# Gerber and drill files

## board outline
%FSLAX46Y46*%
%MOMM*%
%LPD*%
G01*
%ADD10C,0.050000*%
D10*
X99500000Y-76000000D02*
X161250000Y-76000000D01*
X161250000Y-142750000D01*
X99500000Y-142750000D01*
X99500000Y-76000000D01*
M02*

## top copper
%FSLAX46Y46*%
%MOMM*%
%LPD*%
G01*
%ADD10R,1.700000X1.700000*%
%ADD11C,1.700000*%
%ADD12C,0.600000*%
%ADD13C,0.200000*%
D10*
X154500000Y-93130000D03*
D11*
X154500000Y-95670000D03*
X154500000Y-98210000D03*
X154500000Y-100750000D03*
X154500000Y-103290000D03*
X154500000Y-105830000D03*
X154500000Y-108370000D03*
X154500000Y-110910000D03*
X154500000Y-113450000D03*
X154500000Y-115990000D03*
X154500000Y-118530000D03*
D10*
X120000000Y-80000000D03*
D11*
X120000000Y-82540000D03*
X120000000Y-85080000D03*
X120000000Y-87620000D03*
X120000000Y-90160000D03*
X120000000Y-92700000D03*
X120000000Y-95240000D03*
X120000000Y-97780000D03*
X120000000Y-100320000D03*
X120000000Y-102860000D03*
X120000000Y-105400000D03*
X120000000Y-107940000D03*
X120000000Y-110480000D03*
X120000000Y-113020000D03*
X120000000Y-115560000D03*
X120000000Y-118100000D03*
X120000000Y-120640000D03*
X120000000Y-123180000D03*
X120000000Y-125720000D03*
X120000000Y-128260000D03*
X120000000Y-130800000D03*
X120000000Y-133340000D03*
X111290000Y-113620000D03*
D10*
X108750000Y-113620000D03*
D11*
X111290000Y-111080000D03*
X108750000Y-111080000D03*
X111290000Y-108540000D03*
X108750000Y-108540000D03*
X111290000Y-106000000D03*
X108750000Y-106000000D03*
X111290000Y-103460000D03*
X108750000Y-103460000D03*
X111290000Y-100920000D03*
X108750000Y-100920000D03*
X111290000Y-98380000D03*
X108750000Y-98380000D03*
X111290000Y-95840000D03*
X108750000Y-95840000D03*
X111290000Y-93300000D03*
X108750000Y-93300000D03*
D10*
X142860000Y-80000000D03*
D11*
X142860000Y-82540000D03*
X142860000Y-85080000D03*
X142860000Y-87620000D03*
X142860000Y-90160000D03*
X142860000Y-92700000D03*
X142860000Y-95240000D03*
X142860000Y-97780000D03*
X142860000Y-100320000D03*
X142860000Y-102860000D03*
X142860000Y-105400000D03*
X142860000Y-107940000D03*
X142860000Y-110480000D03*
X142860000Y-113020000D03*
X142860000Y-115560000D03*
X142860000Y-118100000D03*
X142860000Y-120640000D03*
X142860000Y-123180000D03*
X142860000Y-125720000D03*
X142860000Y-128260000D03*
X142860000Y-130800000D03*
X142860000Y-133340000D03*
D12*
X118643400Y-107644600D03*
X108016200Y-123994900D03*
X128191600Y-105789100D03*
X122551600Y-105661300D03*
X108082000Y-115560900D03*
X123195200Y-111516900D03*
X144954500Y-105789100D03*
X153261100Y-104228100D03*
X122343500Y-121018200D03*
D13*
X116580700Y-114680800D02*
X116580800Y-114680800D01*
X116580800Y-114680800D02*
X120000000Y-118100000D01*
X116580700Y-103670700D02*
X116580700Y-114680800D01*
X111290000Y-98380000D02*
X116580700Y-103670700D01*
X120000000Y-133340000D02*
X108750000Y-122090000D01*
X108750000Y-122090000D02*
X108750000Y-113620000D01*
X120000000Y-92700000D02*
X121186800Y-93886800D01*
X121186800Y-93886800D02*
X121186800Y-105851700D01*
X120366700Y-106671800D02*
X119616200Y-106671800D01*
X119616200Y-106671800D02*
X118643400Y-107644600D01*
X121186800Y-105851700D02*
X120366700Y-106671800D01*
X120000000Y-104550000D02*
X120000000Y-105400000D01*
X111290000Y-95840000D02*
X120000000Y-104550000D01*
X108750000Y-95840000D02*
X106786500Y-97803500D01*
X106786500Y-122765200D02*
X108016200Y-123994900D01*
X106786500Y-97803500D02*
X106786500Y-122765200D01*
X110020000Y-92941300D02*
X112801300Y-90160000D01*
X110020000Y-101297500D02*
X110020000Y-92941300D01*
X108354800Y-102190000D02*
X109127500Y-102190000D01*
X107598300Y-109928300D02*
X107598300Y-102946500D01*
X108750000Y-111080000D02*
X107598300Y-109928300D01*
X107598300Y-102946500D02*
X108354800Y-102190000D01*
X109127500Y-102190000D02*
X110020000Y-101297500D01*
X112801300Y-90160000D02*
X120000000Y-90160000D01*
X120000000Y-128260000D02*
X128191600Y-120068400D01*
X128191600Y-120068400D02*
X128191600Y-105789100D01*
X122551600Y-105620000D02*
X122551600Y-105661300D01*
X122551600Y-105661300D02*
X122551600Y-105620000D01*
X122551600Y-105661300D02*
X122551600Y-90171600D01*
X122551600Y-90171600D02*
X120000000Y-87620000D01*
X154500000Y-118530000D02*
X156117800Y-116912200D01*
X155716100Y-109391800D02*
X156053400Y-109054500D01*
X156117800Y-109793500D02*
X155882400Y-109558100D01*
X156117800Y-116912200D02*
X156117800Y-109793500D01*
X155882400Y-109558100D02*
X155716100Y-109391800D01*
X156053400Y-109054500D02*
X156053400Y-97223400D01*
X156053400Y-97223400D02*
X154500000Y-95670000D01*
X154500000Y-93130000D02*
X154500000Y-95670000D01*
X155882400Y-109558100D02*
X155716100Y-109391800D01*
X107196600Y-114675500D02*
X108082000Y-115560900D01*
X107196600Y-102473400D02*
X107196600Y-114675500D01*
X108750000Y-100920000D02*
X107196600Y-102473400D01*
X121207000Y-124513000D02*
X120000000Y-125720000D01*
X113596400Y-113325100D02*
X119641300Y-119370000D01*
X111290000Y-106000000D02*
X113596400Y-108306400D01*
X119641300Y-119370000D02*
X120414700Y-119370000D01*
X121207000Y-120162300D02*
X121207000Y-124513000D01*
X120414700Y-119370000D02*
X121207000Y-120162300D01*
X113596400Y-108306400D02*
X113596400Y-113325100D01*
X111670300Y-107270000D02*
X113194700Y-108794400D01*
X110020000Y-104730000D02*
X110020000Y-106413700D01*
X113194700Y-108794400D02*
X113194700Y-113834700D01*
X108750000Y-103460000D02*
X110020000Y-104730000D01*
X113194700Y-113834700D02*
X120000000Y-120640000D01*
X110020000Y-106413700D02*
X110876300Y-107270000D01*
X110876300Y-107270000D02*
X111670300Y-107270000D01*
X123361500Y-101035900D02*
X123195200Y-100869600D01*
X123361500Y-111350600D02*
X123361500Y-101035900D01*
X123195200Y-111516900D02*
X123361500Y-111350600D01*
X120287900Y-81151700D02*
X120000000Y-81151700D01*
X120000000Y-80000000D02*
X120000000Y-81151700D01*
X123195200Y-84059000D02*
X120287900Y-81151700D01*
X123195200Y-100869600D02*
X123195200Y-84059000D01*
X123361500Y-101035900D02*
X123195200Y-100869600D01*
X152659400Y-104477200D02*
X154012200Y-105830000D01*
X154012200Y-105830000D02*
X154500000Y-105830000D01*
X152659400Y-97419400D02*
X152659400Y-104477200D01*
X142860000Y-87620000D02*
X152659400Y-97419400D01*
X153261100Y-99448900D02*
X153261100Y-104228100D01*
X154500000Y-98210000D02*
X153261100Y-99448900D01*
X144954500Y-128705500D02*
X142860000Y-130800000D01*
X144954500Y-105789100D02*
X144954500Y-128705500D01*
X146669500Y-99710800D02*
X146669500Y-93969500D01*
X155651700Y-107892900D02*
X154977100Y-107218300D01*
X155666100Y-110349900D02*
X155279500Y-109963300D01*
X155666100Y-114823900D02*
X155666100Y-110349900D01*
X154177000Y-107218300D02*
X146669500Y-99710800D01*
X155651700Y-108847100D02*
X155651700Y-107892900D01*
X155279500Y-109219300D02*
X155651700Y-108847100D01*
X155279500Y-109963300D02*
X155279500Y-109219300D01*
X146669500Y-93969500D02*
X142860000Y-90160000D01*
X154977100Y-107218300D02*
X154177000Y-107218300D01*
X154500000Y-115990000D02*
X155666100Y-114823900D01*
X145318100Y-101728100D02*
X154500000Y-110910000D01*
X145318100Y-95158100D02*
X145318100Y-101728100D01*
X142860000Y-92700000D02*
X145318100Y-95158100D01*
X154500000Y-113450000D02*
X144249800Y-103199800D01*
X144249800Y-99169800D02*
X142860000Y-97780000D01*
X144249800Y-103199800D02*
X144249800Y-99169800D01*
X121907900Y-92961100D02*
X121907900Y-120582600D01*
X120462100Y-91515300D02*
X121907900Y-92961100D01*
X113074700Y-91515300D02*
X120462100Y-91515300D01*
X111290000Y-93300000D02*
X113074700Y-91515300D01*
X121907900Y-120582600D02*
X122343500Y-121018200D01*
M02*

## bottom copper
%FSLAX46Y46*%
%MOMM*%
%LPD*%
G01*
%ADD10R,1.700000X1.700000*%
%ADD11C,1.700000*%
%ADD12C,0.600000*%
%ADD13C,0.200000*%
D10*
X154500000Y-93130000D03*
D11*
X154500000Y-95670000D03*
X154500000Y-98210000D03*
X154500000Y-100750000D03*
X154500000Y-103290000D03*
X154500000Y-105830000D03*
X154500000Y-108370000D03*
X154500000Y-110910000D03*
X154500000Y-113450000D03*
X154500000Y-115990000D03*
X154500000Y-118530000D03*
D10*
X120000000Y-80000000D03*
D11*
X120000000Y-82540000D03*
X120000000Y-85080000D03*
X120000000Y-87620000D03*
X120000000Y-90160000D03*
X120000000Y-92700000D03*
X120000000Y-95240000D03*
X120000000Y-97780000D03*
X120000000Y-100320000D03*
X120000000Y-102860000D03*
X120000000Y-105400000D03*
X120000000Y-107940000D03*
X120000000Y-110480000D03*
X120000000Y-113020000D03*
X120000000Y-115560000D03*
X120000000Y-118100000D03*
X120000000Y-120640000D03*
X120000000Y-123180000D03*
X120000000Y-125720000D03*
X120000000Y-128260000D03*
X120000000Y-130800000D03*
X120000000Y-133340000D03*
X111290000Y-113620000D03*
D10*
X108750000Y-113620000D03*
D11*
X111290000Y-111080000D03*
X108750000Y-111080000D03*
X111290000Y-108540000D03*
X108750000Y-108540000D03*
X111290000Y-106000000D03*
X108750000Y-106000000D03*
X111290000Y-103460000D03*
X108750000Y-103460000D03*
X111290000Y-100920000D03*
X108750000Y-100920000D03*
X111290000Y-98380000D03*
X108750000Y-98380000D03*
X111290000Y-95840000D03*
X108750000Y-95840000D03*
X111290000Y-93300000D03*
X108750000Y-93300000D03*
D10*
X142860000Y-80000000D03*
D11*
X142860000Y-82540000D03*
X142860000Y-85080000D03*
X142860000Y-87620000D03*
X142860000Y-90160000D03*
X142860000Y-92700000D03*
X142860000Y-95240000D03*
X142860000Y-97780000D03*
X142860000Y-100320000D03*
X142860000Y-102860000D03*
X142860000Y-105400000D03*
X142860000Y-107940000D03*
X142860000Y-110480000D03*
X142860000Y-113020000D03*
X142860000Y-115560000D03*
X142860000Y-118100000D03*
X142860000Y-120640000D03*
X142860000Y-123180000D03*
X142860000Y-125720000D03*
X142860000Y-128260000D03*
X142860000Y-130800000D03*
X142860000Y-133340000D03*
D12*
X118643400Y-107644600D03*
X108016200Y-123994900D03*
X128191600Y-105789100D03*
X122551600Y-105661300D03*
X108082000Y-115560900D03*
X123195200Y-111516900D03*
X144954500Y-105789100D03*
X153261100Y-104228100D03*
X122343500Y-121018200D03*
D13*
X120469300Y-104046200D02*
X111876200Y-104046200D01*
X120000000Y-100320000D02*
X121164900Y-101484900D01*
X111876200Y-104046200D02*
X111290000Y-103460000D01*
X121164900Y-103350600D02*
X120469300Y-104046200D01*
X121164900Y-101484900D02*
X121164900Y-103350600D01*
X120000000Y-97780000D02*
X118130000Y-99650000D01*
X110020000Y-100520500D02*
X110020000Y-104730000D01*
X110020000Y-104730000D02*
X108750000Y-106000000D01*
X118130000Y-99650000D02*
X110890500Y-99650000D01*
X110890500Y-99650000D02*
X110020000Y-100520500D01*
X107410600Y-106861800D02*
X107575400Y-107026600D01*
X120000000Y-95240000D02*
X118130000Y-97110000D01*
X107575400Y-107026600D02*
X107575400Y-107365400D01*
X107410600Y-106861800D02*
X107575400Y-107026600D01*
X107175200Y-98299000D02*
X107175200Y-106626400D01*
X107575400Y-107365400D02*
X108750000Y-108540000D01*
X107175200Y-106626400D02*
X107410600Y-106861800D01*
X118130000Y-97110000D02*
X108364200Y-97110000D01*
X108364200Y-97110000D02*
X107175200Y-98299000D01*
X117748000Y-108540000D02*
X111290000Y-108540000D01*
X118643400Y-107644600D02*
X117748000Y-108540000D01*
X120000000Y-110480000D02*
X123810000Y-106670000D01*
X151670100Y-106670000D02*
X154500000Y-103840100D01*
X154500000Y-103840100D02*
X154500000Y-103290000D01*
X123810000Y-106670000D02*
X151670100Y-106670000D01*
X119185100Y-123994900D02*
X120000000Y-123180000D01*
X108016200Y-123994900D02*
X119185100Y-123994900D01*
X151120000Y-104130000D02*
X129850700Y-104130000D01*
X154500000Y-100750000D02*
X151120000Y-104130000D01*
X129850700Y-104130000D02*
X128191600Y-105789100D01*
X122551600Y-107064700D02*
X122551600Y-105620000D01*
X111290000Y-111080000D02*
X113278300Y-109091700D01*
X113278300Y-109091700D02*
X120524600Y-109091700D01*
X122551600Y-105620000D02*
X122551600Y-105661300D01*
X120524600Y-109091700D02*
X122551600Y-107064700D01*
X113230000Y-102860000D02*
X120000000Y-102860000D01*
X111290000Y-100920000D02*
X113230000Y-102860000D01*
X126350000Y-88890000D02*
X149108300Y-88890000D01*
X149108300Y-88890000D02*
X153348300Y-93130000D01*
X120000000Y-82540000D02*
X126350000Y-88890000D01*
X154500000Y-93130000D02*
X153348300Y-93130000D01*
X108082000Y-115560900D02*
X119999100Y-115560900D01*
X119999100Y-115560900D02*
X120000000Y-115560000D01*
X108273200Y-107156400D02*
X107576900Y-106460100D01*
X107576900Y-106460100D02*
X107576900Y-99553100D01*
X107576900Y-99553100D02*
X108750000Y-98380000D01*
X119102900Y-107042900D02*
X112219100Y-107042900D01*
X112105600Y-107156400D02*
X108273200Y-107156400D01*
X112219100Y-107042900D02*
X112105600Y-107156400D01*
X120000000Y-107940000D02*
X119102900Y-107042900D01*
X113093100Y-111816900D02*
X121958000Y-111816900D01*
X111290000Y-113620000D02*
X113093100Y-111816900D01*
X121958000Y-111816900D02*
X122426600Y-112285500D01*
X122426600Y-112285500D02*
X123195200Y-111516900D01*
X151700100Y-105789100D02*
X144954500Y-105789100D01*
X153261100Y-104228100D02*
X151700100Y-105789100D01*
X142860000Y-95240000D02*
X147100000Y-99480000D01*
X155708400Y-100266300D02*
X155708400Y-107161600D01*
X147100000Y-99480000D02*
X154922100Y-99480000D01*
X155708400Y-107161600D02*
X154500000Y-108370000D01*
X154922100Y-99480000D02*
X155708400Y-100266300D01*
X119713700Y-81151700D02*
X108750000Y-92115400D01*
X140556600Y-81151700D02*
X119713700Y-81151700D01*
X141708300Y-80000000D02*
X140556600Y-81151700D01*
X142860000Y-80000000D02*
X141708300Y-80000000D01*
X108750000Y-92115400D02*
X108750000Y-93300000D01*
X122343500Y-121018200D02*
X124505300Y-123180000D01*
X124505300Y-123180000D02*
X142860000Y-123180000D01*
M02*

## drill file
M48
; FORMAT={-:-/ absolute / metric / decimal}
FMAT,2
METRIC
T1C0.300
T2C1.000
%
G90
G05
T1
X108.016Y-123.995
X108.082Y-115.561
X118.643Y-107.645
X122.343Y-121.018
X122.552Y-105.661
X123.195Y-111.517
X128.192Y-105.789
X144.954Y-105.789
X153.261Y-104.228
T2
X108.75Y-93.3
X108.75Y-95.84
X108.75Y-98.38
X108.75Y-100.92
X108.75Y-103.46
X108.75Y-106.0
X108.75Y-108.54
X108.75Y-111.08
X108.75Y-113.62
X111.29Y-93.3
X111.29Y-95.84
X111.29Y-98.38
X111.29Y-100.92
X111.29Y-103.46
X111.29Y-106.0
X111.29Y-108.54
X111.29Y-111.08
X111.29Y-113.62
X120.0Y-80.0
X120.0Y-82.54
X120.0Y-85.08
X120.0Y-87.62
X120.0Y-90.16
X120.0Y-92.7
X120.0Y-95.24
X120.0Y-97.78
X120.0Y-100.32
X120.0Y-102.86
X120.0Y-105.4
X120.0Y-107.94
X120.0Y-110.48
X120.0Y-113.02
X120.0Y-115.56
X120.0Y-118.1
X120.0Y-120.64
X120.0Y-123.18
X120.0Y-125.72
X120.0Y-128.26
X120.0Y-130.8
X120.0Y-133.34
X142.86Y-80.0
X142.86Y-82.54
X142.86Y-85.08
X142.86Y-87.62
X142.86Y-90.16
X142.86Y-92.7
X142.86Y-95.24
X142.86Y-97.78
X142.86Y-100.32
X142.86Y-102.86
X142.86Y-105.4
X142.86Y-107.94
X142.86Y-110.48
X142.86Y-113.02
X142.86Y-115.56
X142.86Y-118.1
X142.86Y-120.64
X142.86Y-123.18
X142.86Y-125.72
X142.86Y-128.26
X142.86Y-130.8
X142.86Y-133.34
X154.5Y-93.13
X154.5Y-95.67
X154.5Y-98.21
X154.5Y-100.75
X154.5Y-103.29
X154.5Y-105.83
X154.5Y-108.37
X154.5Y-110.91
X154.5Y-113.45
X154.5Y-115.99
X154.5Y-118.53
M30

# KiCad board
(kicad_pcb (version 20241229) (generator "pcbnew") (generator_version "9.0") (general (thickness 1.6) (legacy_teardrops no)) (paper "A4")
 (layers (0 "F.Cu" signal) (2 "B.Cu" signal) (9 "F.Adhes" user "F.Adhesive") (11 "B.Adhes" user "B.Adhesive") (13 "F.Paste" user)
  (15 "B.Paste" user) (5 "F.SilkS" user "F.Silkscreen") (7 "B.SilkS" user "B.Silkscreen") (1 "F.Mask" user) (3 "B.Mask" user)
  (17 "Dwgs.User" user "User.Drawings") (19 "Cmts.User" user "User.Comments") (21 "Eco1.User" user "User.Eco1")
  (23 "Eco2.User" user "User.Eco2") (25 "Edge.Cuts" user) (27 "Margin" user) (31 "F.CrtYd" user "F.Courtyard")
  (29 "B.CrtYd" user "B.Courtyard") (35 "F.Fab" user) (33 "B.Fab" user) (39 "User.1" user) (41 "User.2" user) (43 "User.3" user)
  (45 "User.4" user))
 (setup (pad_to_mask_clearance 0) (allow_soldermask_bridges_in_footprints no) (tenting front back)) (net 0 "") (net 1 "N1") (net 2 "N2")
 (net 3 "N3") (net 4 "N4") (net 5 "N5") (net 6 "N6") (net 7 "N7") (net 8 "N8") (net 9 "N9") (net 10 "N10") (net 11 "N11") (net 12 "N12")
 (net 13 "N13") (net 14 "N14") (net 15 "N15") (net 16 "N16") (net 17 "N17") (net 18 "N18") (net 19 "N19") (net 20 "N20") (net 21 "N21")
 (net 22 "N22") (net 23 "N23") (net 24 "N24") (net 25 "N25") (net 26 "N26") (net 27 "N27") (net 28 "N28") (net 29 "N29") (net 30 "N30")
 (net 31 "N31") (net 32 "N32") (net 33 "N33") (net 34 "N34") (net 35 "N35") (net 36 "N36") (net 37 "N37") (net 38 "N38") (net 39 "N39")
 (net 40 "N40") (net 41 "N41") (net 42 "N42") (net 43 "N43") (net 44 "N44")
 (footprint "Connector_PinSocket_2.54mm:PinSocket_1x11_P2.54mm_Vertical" (layer "F.Cu") (at 154.5 93.13)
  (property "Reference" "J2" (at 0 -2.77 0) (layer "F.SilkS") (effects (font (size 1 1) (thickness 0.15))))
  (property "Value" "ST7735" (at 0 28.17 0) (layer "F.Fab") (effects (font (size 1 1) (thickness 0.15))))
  (pad "1" thru_hole rect (at 0 0) (size 1.7 1.7) (drill 1) (layers "*.Cu" "*.Mask") (remove_unused_layers no) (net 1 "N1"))
  (pad "2" thru_hole circle (at 0 2.54) (size 1.7 1.7) (drill 1) (layers "*.Cu" "*.Mask") (remove_unused_layers no) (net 1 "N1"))
  (pad "3" thru_hole circle (at 0 5.08) (size 1.7 1.7) (drill 1) (layers "*.Cu" "*.Mask") (remove_unused_layers no) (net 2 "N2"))
  (pad "4" thru_hole circle (at 0 7.62) (size 1.7 1.7) (drill 1) (layers "*.Cu" "*.Mask") (remove_unused_layers no) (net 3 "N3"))
  (pad "5" thru_hole circle (at 0 10.16) (size 1.7 1.7) (drill 1) (layers "*.Cu" "*.Mask") (remove_unused_layers no) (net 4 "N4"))
  (pad "6" thru_hole circle (at 0 12.7) (size 1.7 1.7) (drill 1) (layers "*.Cu" "*.Mask") (remove_unused_layers no) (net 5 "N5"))
  (pad "7" thru_hole circle (at 0 15.24) (size 1.7 1.7) (drill 1) (layers "*.Cu" "*.Mask") (remove_unused_layers no) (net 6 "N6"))
  (pad "8" thru_hole circle (at 0 17.78) (size 1.7 1.7) (drill 1) (layers "*.Cu" "*.Mask") (remove_unused_layers no) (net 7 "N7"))
  (pad "9" thru_hole circle (at 0 20.32) (size 1.7 1.7) (drill 1) (layers "*.Cu" "*.Mask") (remove_unused_layers no) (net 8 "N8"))
  (pad "10" thru_hole circle (at 0 22.86) (size 1.7 1.7) (drill 1) (layers "*.Cu" "*.Mask") (remove_unused_layers no) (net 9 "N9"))
  (pad "11" thru_hole circle (at 0 25.4) (size 1.7 1.7) (drill 1) (layers "*.Cu" "*.Mask") (remove_unused_layers no) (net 1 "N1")))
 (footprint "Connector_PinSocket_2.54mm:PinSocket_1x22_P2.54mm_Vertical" (layer "F.Cu") (at 120 80)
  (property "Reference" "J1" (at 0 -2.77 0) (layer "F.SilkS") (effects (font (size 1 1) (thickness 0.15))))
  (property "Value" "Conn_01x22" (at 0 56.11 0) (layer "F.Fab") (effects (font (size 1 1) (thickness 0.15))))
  (pad "1" thru_hole rect (at 0 0) (size 1.7 1.7) (drill 1) (layers "*.Cu" "*.Mask") (remove_unused_layers no) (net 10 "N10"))
  (pad "2" thru_hole circle (at 0 2.54) (size 1.7 1.7) (drill 1) (layers "*.Cu" "*.Mask") (remove_unused_layers no) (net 1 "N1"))
  (pad "3" thru_hole circle (at 0 5.08) (size 1.7 1.7) (drill 1) (layers "*.Cu" "*.Mask") (remove_unused_layers no) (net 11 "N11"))
  (pad "4" thru_hole circle (at 0 7.62) (size 1.7 1.7) (drill 1) (layers "*.Cu" "*.Mask") (remove_unused_layers no) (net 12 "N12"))
  (pad "5" thru_hole circle (at 0 10.16) (size 1.7 1.7) (drill 1) (layers "*.Cu" "*.Mask") (remove_unused_layers no) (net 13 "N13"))
  (pad "6" thru_hole circle (at 0 12.7) (size 1.7 1.7) (drill 1) (layers "*.Cu" "*.Mask") (remove_unused_layers no) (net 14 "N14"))
  (pad "7" thru_hole circle (at 0 15.24) (size 1.7 1.7) (drill 1) (layers "*.Cu" "*.Mask") (remove_unused_layers no) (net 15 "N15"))
  (pad "8" thru_hole circle (at 0 17.78) (size 1.7 1.7) (drill 1) (layers "*.Cu" "*.Mask") (remove_unused_layers no) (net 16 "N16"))
  (pad "9" thru_hole circle (at 0 20.32) (size 1.7 1.7) (drill 1) (layers "*.Cu" "*.Mask") (remove_unused_layers no) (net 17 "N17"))
  (pad "10" thru_hole circle (at 0 22.86) (size 1.7 1.7) (drill 1) (layers "*.Cu" "*.Mask") (remove_unused_layers no) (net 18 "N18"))
  (pad "11" thru_hole circle (at 0 25.4) (size 1.7 1.7) (drill 1) (layers "*.Cu" "*.Mask") (remove_unused_layers no) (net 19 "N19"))
  (pad "12" thru_hole circle (at 0 27.94) (size 1.7 1.7) (drill 1) (layers "*.Cu" "*.Mask") (remove_unused_layers no) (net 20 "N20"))
  (pad "13" thru_hole circle (at 0 30.48) (size 1.7 1.7) (drill 1) (layers "*.Cu" "*.Mask") (remove_unused_layers no) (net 4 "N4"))
  (pad "14" thru_hole circle (at 0 33.02) (size 1.7 1.7) (drill 1) (layers "*.Cu" "*.Mask") (remove_unused_layers no) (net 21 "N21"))
  (pad "15" thru_hole circle (at 0 35.56) (size 1.7 1.7) (drill 1) (layers "*.Cu" "*.Mask") (remove_unused_layers no) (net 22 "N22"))
  (pad "16" thru_hole circle (at 0 38.1) (size 1.7 1.7) (drill 1) (layers "*.Cu" "*.Mask") (remove_unused_layers no) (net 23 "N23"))
  (pad "17" thru_hole circle (at 0 40.64) (size 1.7 1.7) (drill 1) (layers "*.Cu" "*.Mask") (remove_unused_layers no) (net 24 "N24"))
  (pad "18" thru_hole circle (at 0 43.18) (size 1.7 1.7) (drill 1) (layers "*.Cu" "*.Mask") (remove_unused_layers no) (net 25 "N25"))
  (pad "19" thru_hole circle (at 0 45.72) (size 1.7 1.7) (drill 1) (layers "*.Cu" "*.Mask") (remove_unused_layers no) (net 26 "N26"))
  (pad "20" thru_hole circle (at 0 48.26) (size 1.7 1.7) (drill 1) (layers "*.Cu" "*.Mask") (remove_unused_layers no) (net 3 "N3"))
  (pad "21" thru_hole circle (at 0 50.8) (size 1.7 1.7) (drill 1) (layers "*.Cu" "*.Mask") (remove_unused_layers no) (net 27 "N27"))
  (pad "22" thru_hole circle (at 0 53.34) (size 1.7 1.7) (drill 1) (layers "*.Cu" "*.Mask") (remove_unused_layers no) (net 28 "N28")))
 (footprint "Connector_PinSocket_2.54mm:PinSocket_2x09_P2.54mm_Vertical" (layer "F.Cu") (at 108.75 113.62 180)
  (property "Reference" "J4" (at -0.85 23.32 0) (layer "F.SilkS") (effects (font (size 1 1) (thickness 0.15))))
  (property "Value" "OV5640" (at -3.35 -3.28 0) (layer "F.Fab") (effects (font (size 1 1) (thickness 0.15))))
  (pad "1" thru_hole circle (at -2.54 0 180) (size 1.7 1.7) (drill 1) (layers "*.Cu" "*.Mask") (remove_unused_layers no) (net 10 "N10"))
  (pad "2" thru_hole rect (at 0 0 180) (size 1.7 1.7) (drill 1) (layers "*.Cu" "*.Mask") (remove_unused_layers no) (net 28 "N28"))
  (pad "3" thru_hole circle (at -2.54 2.54 180) (size 1.7 1.7) (drill 1) (layers "*.Cu" "*.Mask") (remove_unused_layers no) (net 12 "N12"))
  (pad "4" thru_hole circle (at 0 2.54 180) (size 1.7 1.7) (drill 1) (layers "*.Cu" "*.Mask") (remove_unused_layers no) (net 13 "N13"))
  (pad "5" thru_hole circle (at -2.54 5.08 180) (size 1.7 1.7) (drill 1) (layers "*.Cu" "*.Mask") (remove_unused_layers no) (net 14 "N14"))
  (pad "6" thru_hole circle (at 0 5.08 180) (size 1.7 1.7) (drill 1) (layers "*.Cu" "*.Mask") (remove_unused_layers no) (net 15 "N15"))
  (pad "7" thru_hole circle (at -2.54 7.62 180) (size 1.7 1.7) (drill 1) (layers "*.Cu" "*.Mask") (remove_unused_layers no) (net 26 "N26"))
  (pad "8" thru_hole circle (at 0 7.62 180) (size 1.7 1.7) (drill 1) (layers "*.Cu" "*.Mask") (remove_unused_layers no) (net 16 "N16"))
  (pad "9" thru_hole circle (at -2.54 10.16 180) (size 1.7 1.7) (drill 1) (layers "*.Cu" "*.Mask") (remove_unused_layers no) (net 17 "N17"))
  (pad "10" thru_hole circle (at 0 10.16 180) (size 1.7 1.7) (drill 1) (layers "*.Cu" "*.Mask") (remove_unused_layers no) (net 24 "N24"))
  (pad "11" thru_hole circle (at -2.54 12.7 180) (size 1.7 1.7) (drill 1) (layers "*.Cu" "*.Mask") (remove_unused_layers no) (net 18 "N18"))
  (pad "12" thru_hole circle (at 0 12.7 180) (size 1.7 1.7) (drill 1) (layers "*.Cu" "*.Mask") (remove_unused_layers no) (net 22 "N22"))
  (pad "13" thru_hole circle (at -2.54 15.24 180) (size 1.7 1.7) (drill 1) (layers "*.Cu" "*.Mask") (remove_unused_layers no) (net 23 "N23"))
  (pad "14" thru_hole circle (at 0 15.24 180) (size 1.7 1.7) (drill 1) (layers "*.Cu" "*.Mask") (remove_unused_layers no) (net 20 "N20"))
  (pad "15" thru_hole circle (at -2.54 17.78 180) (size 1.7 1.7) (drill 1) (layers "*.Cu" "*.Mask") (remove_unused_layers no) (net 19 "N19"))
  (pad "16" thru_hole circle (at 0 17.78 180) (size 1.7 1.7) (drill 1) (layers "*.Cu" "*.Mask") (remove_unused_layers no) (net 25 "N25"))
  (pad "17" thru_hole circle (at -2.54 20.32 180) (size 1.7 1.7) (drill 1) (layers "*.Cu" "*.Mask") (remove_unused_layers no) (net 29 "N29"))
  (pad "18" thru_hole circle (at 0 20.32 180) (size 1.7 1.7) (drill 1) (layers "*.Cu" "*.Mask") (remove_unused_layers no) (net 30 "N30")))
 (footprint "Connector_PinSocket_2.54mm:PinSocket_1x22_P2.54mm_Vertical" (layer "F.Cu") (at 142.86 80)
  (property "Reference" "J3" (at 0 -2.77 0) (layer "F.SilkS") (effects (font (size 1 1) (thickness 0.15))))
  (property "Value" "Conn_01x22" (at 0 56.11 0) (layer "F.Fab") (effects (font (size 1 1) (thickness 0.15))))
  (pad "1" thru_hole rect (at 0 0) (size 1.7 1.7) (drill 1) (layers "*.Cu" "*.Mask") (remove_unused_layers no) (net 30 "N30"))
  (pad "2" thru_hole circle (at 0 2.54) (size 1.7 1.7) (drill 1) (layers "*.Cu" "*.Mask") (remove_unused_layers no) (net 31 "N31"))
  (pad "3" thru_hole circle (at 0 5.08) (size 1.7 1.7) (drill 1) (layers "*.Cu" "*.Mask") (remove_unused_layers no) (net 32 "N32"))
  (pad "4" thru_hole circle (at 0 7.62) (size 1.7 1.7) (drill 1) (layers "*.Cu" "*.Mask") (remove_unused_layers no) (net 5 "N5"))
  (pad "5" thru_hole circle (at 0 10.16) (size 1.7 1.7) (drill 1) (layers "*.Cu" "*.Mask") (remove_unused_layers no) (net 9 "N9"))
  (pad "6" thru_hole circle (at 0 12.7) (size 1.7 1.7) (drill 1) (layers "*.Cu" "*.Mask") (remove_unused_layers no) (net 7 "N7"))
  (pad "7" thru_hole circle (at 0 15.24) (size 1.7 1.7) (drill 1) (layers "*.Cu" "*.Mask") (remove_unused_layers no) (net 6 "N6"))
  (pad "8" thru_hole circle (at 0 17.78) (size 1.7 1.7) (drill 1) (layers "*.Cu" "*.Mask") (remove_unused_layers no) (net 8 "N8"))
  (pad "9" thru_hole circle (at 0 20.32) (size 1.7 1.7) (drill 1) (layers "*.Cu" "*.Mask") (remove_unused_layers no) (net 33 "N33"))
  (pad "10" thru_hole circle (at 0 22.86) (size 1.7 1.7) (drill 1) (layers "*.Cu" "*.Mask") (remove_unused_layers no) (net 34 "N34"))
  (pad "11" thru_hole circle (at 0 25.4) (size 1.7 1.7) (drill 1) (layers "*.Cu" "*.Mask") (remove_unused_layers no) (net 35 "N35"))
  (pad "12" thru_hole circle (at 0 27.94) (size 1.7 1.7) (drill 1) (layers "*.Cu" "*.Mask") (remove_unused_layers no) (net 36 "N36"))
  (pad "13" thru_hole circle (at 0 30.48) (size 1.7 1.7) (drill 1) (layers "*.Cu" "*.Mask") (remove_unused_layers no) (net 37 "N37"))
  (pad "14" thru_hole circle (at 0 33.02) (size 1.7 1.7) (drill 1) (layers "*.Cu" "*.Mask") (remove_unused_layers no) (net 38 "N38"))
  (pad "15" thru_hole circle (at 0 35.56) (size 1.7 1.7) (drill 1) (layers "*.Cu" "*.Mask") (remove_unused_layers no) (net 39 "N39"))
  (pad "16" thru_hole circle (at 0 38.1) (size 1.7 1.7) (drill 1) (layers "*.Cu" "*.Mask") (remove_unused_layers no) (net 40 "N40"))
  (pad "17" thru_hole circle (at 0 40.64) (size 1.7 1.7) (drill 1) (layers "*.Cu" "*.Mask") (remove_unused_layers no) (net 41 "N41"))
  (pad "18" thru_hole circle (at 0 43.18) (size 1.7 1.7) (drill 1) (layers "*.Cu" "*.Mask") (remove_unused_layers no) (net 29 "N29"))
  (pad "19" thru_hole circle (at 0 45.72) (size 1.7 1.7) (drill 1) (layers "*.Cu" "*.Mask") (remove_unused_layers no) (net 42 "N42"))
  (pad "20" thru_hole circle (at 0 48.26) (size 1.7 1.7) (drill 1) (layers "*.Cu" "*.Mask") (remove_unused_layers no) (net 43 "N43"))
  (pad "21" thru_hole circle (at 0 50.8) (size 1.7 1.7) (drill 1) (layers "*.Cu" "*.Mask") (remove_unused_layers no) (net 2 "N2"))
  (pad "22" thru_hole circle (at 0 53.34) (size 1.7 1.7) (drill 1) (layers "*.Cu" "*.Mask") (remove_unused_layers no) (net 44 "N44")))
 (gr_rect (start 99.5 76) (end 161.25 142.75) (stroke (width 0.05) (type default)) (fill no) (layer "Edge.Cuts"))
 (segment (start 120.4693 104.0462) (end 111.8762 104.0462) (width 0.2) (layer "B.Cu") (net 17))
 (segment (start 120 100.32) (end 121.1649 101.4849) (width 0.2) (layer "B.Cu") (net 17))
 (segment (start 111.8762 104.0462) (end 111.29 103.46) (width 0.2) (layer "B.Cu") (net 17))
 (segment (start 121.1649 103.3506) (end 120.4693 104.0462) (width 0.2) (layer "B.Cu") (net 17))
 (segment (start 121.1649 101.4849) (end 121.1649 103.3506) (width 0.2) (layer "B.Cu") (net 17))
 (segment (start 120 97.78) (end 118.13 99.65) (width 0.2) (layer "B.Cu") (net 16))
 (segment (start 110.02 100.5205) (end 110.02 104.73) (width 0.2) (layer "B.Cu") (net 16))
 (segment (start 110.02 104.73) (end 108.75 106) (width 0.2) (layer "B.Cu") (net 16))
 (segment (start 118.13 99.65) (end 110.8905 99.65) (width 0.2) (layer "B.Cu") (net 16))
 (segment (start 110.8905 99.65) (end 110.02 100.5205) (width 0.2) (layer "B.Cu") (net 16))
 (segment (start 107.4106 106.8618) (end 107.5754 107.0266) (width 0.2) (layer "B.Cu") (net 15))
 (segment (start 120 95.24) (end 118.13 97.11) (width 0.2) (layer "B.Cu") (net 15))
 (segment (start 107.5754 107.0266) (end 107.5754 107.3654) (width 0.2) (layer "B.Cu") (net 15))
 (segment (start 107.4106 106.8618) (end 107.5754 107.0266) (width 0.2) (layer "B.Cu") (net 15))
 (segment (start 107.1752 98.299) (end 107.1752 106.6264) (width 0.2) (layer "B.Cu") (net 15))
 (segment (start 107.5754 107.3654) (end 108.75 108.54) (width 0.2) (layer "B.Cu") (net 15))
 (segment (start 107.1752 106.6264) (end 107.4106 106.8618) (width 0.2) (layer "B.Cu") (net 15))
 (segment (start 118.13 97.11) (end 108.3642 97.11) (width 0.2) (layer "B.Cu") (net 15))
 (segment (start 108.3642 97.11) (end 107.1752 98.299) (width 0.2) (layer "B.Cu") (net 15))
 (segment (start 116.5807 114.6808) (end 116.5808 114.6808) (width 0.2) (layer "F.Cu") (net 23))
 (segment (start 116.5808 114.6808) (end 120 118.1) (width 0.2) (layer "F.Cu") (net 23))
 (segment (start 116.5807 103.6707) (end 116.5807 114.6808) (width 0.2) (layer "F.Cu") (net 23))
 (segment (start 111.29 98.38) (end 116.5807 103.6707) (width 0.2) (layer "F.Cu") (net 23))
 (segment (start 120 133.34) (end 108.75 122.09) (width 0.2) (layer "F.Cu") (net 28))
 (segment (start 108.75 122.09) (end 108.75 113.62) (width 0.2) (layer "F.Cu") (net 28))
 (segment (start 120 92.7) (end 121.1868 93.8868) (width 0.2) (layer "F.Cu") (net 14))
 (segment (start 121.1868 93.8868) (end 121.1868 105.8517) (width 0.2) (layer "F.Cu") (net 14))
 (segment (start 120.3667 106.6718) (end 119.6162 106.6718) (width 0.2) (layer "F.Cu") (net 14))
 (segment (start 119.6162 106.6718) (end 118.6434 107.6446) (width 0.2) (layer "F.Cu") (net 14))
 (segment (start 121.1868 105.8517) (end 120.3667 106.6718) (width 0.2) (layer "F.Cu") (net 14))
 (via (at 118.6434 107.6446) (size 0.6) (drill 0.3) (layers "F.Cu" "B.Cu") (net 14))
 (segment (start 117.748 108.54) (end 111.29 108.54) (width 0.2) (layer "B.Cu") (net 14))
 (segment (start 118.6434 107.6446) (end 117.748 108.54) (width 0.2) (layer "B.Cu") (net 14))
 (segment (start 120 110.48) (end 123.81 106.67) (width 0.2) (layer "B.Cu") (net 4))
 (segment (start 151.6701 106.67) (end 154.5 103.8401) (width 0.2) (layer "B.Cu") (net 4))
 (segment (start 154.5 103.8401) (end 154.5 103.29) (width 0.2) (layer "B.Cu") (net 4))
 (segment (start 123.81 106.67) (end 151.6701 106.67) (width 0.2) (layer "B.Cu") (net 4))
 (segment (start 120 104.55) (end 120 105.4) (width 0.2) (layer "F.Cu") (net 19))
 (segment (start 111.29 95.84) (end 120 104.55) (width 0.2) (layer "F.Cu") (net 19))
 (segment (start 108.75 95.84) (end 106.7865 97.8035) (width 0.2) (layer "F.Cu") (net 25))
 (segment (start 106.7865 122.7652) (end 108.0162 123.9949) (width 0.2) (layer "F.Cu") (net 25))
 (segment (start 106.7865 97.8035) (end 106.7865 122.7652) (width 0.2) (layer "F.Cu") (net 25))
 (via (at 108.0162 123.9949) (size 0.6) (drill 0.3) (layers "F.Cu" "B.Cu") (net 25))
 (segment (start 119.1851 123.9949) (end 120 123.18) (width 0.2) (layer "B.Cu") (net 25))
 (segment (start 108.0162 123.9949) (end 119.1851 123.9949) (width 0.2) (layer "B.Cu") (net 25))
 (segment (start 110.02 92.9413) (end 112.8013 90.16) (width 0.2) (layer "F.Cu") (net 13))
 (segment (start 110.02 101.2975) (end 110.02 92.9413) (width 0.2) (layer "F.Cu") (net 13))
 (segment (start 108.3548 102.19) (end 109.1275 102.19) (width 0.2) (layer "F.Cu") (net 13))
 (segment (start 107.5983 109.9283) (end 107.5983 102.9465) (width 0.2) (layer "F.Cu") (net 13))
 (segment (start 108.75 111.08) (end 107.5983 109.9283) (width 0.2) (layer "F.Cu") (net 13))
 (segment (start 107.5983 102.9465) (end 108.3548 102.19) (width 0.2) (layer "F.Cu") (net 13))
 (segment (start 109.1275 102.19) (end 110.02 101.2975) (width 0.2) (layer "F.Cu") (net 13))
 (segment (start 112.8013 90.16) (end 120 90.16) (width 0.2) (layer "F.Cu") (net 13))
 (segment (start 120 128.26) (end 128.1916 120.0684) (width 0.2) (layer "F.Cu") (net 3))
 (segment (start 128.1916 120.0684) (end 128.1916 105.7891) (width 0.2) (layer "F.Cu") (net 3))
 (via (at 128.1916 105.7891) (size 0.6) (drill 0.3) (layers "F.Cu" "B.Cu") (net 3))
 (segment (start 151.12 104.13) (end 129.8507 104.13) (width 0.2) (layer "B.Cu") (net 3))
 (segment (start 154.5 100.75) (end 151.12 104.13) (width 0.2) (layer "B.Cu") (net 3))
 (segment (start 129.8507 104.13) (end 128.1916 105.7891) (width 0.2) (layer "B.Cu") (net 3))
 (segment (start 122.5516 105.62) (end 122.5516 105.6613) (width 0.2) (layer "F.Cu") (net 12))
 (segment (start 122.5516 105.6613) (end 122.5516 105.62) (width 0.2) (layer "F.Cu") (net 12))
 (segment (start 122.5516 105.6613) (end 122.5516 90.1716) (width 0.2) (layer "F.Cu") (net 12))
 (segment (start 122.5516 90.1716) (end 120 87.62) (width 0.2) (layer "F.Cu") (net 12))
 (via (at 122.5516 105.6613) (size 0.6) (drill 0.3) (layers "F.Cu" "B.Cu") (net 12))
 (segment (start 122.5516 107.0647) (end 122.5516 105.62) (width 0.2) (layer "B.Cu") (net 12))
 (segment (start 111.29 111.08) (end 113.2783 109.0917) (width 0.2) (layer "B.Cu") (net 12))
 (segment (start 113.2783 109.0917) (end 120.5246 109.0917) (width 0.2) (layer "B.Cu") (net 12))
 (segment (start 122.5516 105.62) (end 122.5516 105.6613) (width 0.2) (layer "B.Cu") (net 12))
 (segment (start 120.5246 109.0917) (end 122.5516 107.0647) (width 0.2) (layer "B.Cu") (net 12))
 (segment (start 113.23 102.86) (end 120 102.86) (width 0.2) (layer "B.Cu") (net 18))
 (segment (start 111.29 100.92) (end 113.23 102.86) (width 0.2) (layer "B.Cu") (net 18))
 (segment (start 154.5 118.53) (end 156.1178 116.9122) (width 0.2) (layer "F.Cu") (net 1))
 (segment (start 155.7161 109.3918) (end 156.0534 109.0545) (width 0.2) (layer "F.Cu") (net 1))
 (segment (start 156.1178 109.7935) (end 155.8824 109.5581) (width 0.2) (layer "F.Cu") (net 1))
 (segment (start 156.1178 116.9122) (end 156.1178 109.7935) (width 0.2) (layer "F.Cu") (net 1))
 (segment (start 155.8824 109.5581) (end 155.7161 109.3918) (width 0.2) (layer "F.Cu") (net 1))
 (segment (start 156.0534 109.0545) (end 156.0534 97.2234) (width 0.2) (layer "F.Cu") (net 1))
 (segment (start 156.0534 97.2234) (end 154.5 95.67) (width 0.2) (layer "F.Cu") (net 1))
 (segment (start 154.5 93.13) (end 154.5 95.67) (width 0.2) (layer "F.Cu") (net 1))
 (segment (start 155.8824 109.5581) (end 155.7161 109.3918) (width 0.2) (layer "F.Cu") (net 1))
 (segment (start 126.35 88.89) (end 149.1083 88.89) (width 0.2) (layer "B.Cu") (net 1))
 (segment (start 149.1083 88.89) (end 153.3483 93.13) (width 0.2) (layer "B.Cu") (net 1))
 (segment (start 120 82.54) (end 126.35 88.89) (width 0.2) (layer "B.Cu") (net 1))
 (segment (start 154.5 93.13) (end 153.3483 93.13) (width 0.2) (layer "B.Cu") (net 1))
 (segment (start 107.1966 114.6755) (end 108.082 115.5609) (width 0.2) (layer "F.Cu") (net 22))
 (segment (start 107.1966 102.4734) (end 107.1966 114.6755) (width 0.2) (layer "F.Cu") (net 22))
 (segment (start 108.75 100.92) (end 107.1966 102.4734) (width 0.2) (layer "F.Cu") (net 22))
 (via (at 108.082 115.5609) (size 0.6) (drill 0.3) (layers "F.Cu" "B.Cu") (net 22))
 (segment (start 108.082 115.5609) (end 119.9991 115.5609) (width 0.2) (layer "B.Cu") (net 22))
 (segment (start 119.9991 115.5609) (end 120 115.56) (width 0.2) (layer "B.Cu") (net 22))
 (segment (start 108.2732 107.1564) (end 107.5769 106.4601) (width 0.2) (layer "B.Cu") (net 20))
 (segment (start 107.5769 106.4601) (end 107.5769 99.5531) (width 0.2) (layer "B.Cu") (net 20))
 (segment (start 107.5769 99.5531) (end 108.75 98.38) (width 0.2) (layer "B.Cu") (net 20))
 (segment (start 119.1029 107.0429) (end 112.2191 107.0429) (width 0.2) (layer "B.Cu") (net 20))
 (segment (start 112.1056 107.1564) (end 108.2732 107.1564) (width 0.2) (layer "B.Cu") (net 20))
 (segment (start 112.2191 107.0429) (end 112.1056 107.1564) (width 0.2) (layer "B.Cu") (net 20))
 (segment (start 120 107.94) (end 119.1029 107.0429) (width 0.2) (layer "B.Cu") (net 20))
 (segment (start 121.207 124.513) (end 120 125.72) (width 0.2) (layer "F.Cu") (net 26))
 (segment (start 113.5964 113.3251) (end 119.6413 119.37) (width 0.2) (layer "F.Cu") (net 26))
 (segment (start 111.29 106) (end 113.5964 108.3064) (width 0.2) (layer "F.Cu") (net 26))
 (segment (start 119.6413 119.37) (end 120.4147 119.37) (width 0.2) (layer "F.Cu") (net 26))
 (segment (start 121.207 120.1623) (end 121.207 124.513) (width 0.2) (layer "F.Cu") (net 26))
 (segment (start 120.4147 119.37) (end 121.207 120.1623) (width 0.2) (layer "F.Cu") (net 26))
 (segment (start 113.5964 108.3064) (end 113.5964 113.3251) (width 0.2) (layer "F.Cu") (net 26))
 (segment (start 111.6703 107.27) (end 113.1947 108.7944) (width 0.2) (layer "F.Cu") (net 24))
 (segment (start 110.02 104.73) (end 110.02 106.4137) (width 0.2) (layer "F.Cu") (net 24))
 (segment (start 113.1947 108.7944) (end 113.1947 113.8347) (width 0.2) (layer "F.Cu") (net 24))
 (segment (start 108.75 103.46) (end 110.02 104.73) (width 0.2) (layer "F.Cu") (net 24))
 (segment (start 113.1947 113.8347) (end 120 120.64) (width 0.2) (layer "F.Cu") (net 24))
 (segment (start 110.02 106.4137) (end 110.8763 107.27) (width 0.2) (layer "F.Cu") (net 24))
 (segment (start 110.8763 107.27) (end 111.6703 107.27) (width 0.2) (layer "F.Cu") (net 24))
 (segment (start 123.3615 101.0359) (end 123.1952 100.8696) (width 0.2) (layer "F.Cu") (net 10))
 (segment (start 123.3615 111.3506) (end 123.3615 101.0359) (width 0.2) (layer "F.Cu") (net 10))
 (segment (start 123.1952 111.5169) (end 123.3615 111.3506) (width 0.2) (layer "F.Cu") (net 10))
 (segment (start 120.2879 81.1517) (end 120 81.1517) (width 0.2) (layer "F.Cu") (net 10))
 (segment (start 120 80) (end 120 81.1517) (width 0.2) (layer "F.Cu") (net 10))
 (segment (start 123.1952 84.059) (end 120.2879 81.1517) (width 0.2) (layer "F.Cu") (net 10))
 (segment (start 123.1952 100.8696) (end 123.1952 84.059) (width 0.2) (layer "F.Cu") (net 10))
 (segment (start 123.3615 101.0359) (end 123.1952 100.8696) (width 0.2) (layer "F.Cu") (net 10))
 (via (at 123.1952 111.5169) (size 0.6) (drill 0.3) (layers "F.Cu" "B.Cu") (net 10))
 (segment (start 113.0931 111.8169) (end 121.958 111.8169) (width 0.2) (layer "B.Cu") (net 10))
 (segment (start 111.29 113.62) (end 113.0931 111.8169) (width 0.2) (layer "B.Cu") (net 10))
 (segment (start 121.958 111.8169) (end 122.4266 112.2855) (width 0.2) (layer "B.Cu") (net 10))
 (segment (start 122.4266 112.2855) (end 123.1952 111.5169) (width 0.2) (layer "B.Cu") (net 10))
 (segment (start 152.6594 104.4772) (end 154.0122 105.83) (width 0.2) (layer "F.Cu") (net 5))
 (segment (start 154.0122 105.83) (end 154.5 105.83) (width 0.2) (layer "F.Cu") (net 5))
 (segment (start 152.6594 97.4194) (end 152.6594 104.4772) (width 0.2) (layer "F.Cu") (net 5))
 (segment (start 142.86 87.62) (end 152.6594 97.4194) (width 0.2) (layer "F.Cu") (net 5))
 (segment (start 153.2611 99.4489) (end 153.2611 104.2281) (width 0.2) (layer "F.Cu") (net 2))
 (segment (start 154.5 98.21) (end 153.2611 99.4489) (width 0.2) (layer "F.Cu") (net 2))
 (segment (start 144.9545 128.7055) (end 142.86 130.8) (width 0.2) (layer "F.Cu") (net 2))
 (segment (start 144.9545 105.7891) (end 144.9545 128.7055) (width 0.2) (layer "F.Cu") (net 2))
 (via (at 144.9545 105.7891) (size 0.6) (drill 0.3) (layers "F.Cu" "B.Cu") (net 2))
 (via (at 153.2611 104.2281) (size 0.6) (drill 0.3) (layers "F.Cu" "B.Cu") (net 2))
 (segment (start 151.7001 105.7891) (end 144.9545 105.7891) (width 0.2) (layer "B.Cu") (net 2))
 (segment (start 153.2611 104.2281) (end 151.7001 105.7891) (width 0.2) (layer "B.Cu") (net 2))
 (segment (start 146.6695 99.7108) (end 146.6695 93.9695) (width 0.2) (layer "F.Cu") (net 9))
 (segment (start 155.6517 107.8929) (end 154.9771 107.2183) (width 0.2) (layer "F.Cu") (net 9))
 (segment (start 155.6661 110.3499) (end 155.2795 109.9633) (width 0.2) (layer "F.Cu") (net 9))
 (segment (start 155.6661 114.8239) (end 155.6661 110.3499) (width 0.2) (layer "F.Cu") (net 9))
 (segment (start 154.177 107.2183) (end 146.6695 99.7108) (width 0.2) (layer "F.Cu") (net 9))
 (segment (start 155.6517 108.8471) (end 155.6517 107.8929) (width 0.2) (layer "F.Cu") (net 9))
 (segment (start 155.2795 109.2193) (end 155.6517 108.8471) (width 0.2) (layer "F.Cu") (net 9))
 (segment (start 155.2795 109.9633) (end 155.2795 109.2193) (width 0.2) (layer "F.Cu") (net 9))
 (segment (start 146.6695 93.9695) (end 142.86 90.16) (width 0.2) (layer "F.Cu") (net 9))
 (segment (start 154.9771 107.2183) (end 154.177 107.2183) (width 0.2) (layer "F.Cu") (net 9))
 (segment (start 154.5 115.99) (end 155.6661 114.8239) (width 0.2) (layer "F.Cu") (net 9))
 (segment (start 145.3181 101.7281) (end 154.5 110.91) (width 0.2) (layer "F.Cu") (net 7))
 (segment (start 145.3181 95.1581) (end 145.3181 101.7281) (width 0.2) (layer "F.Cu") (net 7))
 (segment (start 142.86 92.7) (end 145.3181 95.1581) (width 0.2) (layer "F.Cu") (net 7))
 (segment (start 154.5 113.45) (end 144.2498 103.1998) (width 0.2) (layer "F.Cu") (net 8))
 (segment (start 144.2498 99.1698) (end 142.86 97.78) (width 0.2) (layer "F.Cu") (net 8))
 (segment (start 144.2498 103.1998) (end 144.2498 99.1698) (width 0.2) (layer "F.Cu") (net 8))
 (segment (start 142.86 95.24) (end 147.1 99.48) (width 0.2) (layer "B.Cu") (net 6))
 (segment (start 155.7084 100.2663) (end 155.7084 107.1616) (width 0.2) (layer "B.Cu") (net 6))
 (segment (start 147.1 99.48) (end 154.9221 99.48) (width 0.2) (layer "B.Cu") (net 6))
 (segment (start 155.7084 107.1616) (end 154.5 108.37) (width 0.2) (layer "B.Cu") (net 6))
 (segment (start 154.9221 99.48) (end 155.7084 100.2663) (width 0.2) (layer "B.Cu") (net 6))
 (segment (start 119.7137 81.1517) (end 108.75 92.1154) (width 0.2) (layer "B.Cu") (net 30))
 (segment (start 140.5566 81.1517) (end 119.7137 81.1517) (width 0.2) (layer "B.Cu") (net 30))
 (segment (start 141.7083 80) (end 140.5566 81.1517) (width 0.2) (layer "B.Cu") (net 30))
 (segment (start 142.86 80) (end 141.7083 80) (width 0.2) (layer "B.Cu") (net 30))
 (segment (start 108.75 92.1154) (end 108.75 93.3) (width 0.2) (layer "B.Cu") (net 30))
 (segment (start 121.9079 92.9611) (end 121.9079 120.5826) (width 0.2) (layer "F.Cu") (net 29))
 (segment (start 120.4621 91.5153) (end 121.9079 92.9611) (width 0.2) (layer "F.Cu") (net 29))
 (segment (start 113.0747 91.5153) (end 120.4621 91.5153) (width 0.2) (layer "F.Cu") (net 29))
 (segment (start 111.29 93.3) (end 113.0747 91.5153) (width 0.2) (layer "F.Cu") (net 29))
 (segment (start 121.9079 120.5826) (end 122.3435 121.0182) (width 0.2) (layer "F.Cu") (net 29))
 (via (at 122.3435 121.0182) (size 0.6) (drill 0.3) (layers "F.Cu" "B.Cu") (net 29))
 (segment (start 122.3435 121.0182) (end 124.5053 123.18) (width 0.2) (layer "B.Cu") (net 29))
 (segment (start 124.5053 123.18) (end 142.86 123.18) (width 0.2) (layer "B.Cu") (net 29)))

